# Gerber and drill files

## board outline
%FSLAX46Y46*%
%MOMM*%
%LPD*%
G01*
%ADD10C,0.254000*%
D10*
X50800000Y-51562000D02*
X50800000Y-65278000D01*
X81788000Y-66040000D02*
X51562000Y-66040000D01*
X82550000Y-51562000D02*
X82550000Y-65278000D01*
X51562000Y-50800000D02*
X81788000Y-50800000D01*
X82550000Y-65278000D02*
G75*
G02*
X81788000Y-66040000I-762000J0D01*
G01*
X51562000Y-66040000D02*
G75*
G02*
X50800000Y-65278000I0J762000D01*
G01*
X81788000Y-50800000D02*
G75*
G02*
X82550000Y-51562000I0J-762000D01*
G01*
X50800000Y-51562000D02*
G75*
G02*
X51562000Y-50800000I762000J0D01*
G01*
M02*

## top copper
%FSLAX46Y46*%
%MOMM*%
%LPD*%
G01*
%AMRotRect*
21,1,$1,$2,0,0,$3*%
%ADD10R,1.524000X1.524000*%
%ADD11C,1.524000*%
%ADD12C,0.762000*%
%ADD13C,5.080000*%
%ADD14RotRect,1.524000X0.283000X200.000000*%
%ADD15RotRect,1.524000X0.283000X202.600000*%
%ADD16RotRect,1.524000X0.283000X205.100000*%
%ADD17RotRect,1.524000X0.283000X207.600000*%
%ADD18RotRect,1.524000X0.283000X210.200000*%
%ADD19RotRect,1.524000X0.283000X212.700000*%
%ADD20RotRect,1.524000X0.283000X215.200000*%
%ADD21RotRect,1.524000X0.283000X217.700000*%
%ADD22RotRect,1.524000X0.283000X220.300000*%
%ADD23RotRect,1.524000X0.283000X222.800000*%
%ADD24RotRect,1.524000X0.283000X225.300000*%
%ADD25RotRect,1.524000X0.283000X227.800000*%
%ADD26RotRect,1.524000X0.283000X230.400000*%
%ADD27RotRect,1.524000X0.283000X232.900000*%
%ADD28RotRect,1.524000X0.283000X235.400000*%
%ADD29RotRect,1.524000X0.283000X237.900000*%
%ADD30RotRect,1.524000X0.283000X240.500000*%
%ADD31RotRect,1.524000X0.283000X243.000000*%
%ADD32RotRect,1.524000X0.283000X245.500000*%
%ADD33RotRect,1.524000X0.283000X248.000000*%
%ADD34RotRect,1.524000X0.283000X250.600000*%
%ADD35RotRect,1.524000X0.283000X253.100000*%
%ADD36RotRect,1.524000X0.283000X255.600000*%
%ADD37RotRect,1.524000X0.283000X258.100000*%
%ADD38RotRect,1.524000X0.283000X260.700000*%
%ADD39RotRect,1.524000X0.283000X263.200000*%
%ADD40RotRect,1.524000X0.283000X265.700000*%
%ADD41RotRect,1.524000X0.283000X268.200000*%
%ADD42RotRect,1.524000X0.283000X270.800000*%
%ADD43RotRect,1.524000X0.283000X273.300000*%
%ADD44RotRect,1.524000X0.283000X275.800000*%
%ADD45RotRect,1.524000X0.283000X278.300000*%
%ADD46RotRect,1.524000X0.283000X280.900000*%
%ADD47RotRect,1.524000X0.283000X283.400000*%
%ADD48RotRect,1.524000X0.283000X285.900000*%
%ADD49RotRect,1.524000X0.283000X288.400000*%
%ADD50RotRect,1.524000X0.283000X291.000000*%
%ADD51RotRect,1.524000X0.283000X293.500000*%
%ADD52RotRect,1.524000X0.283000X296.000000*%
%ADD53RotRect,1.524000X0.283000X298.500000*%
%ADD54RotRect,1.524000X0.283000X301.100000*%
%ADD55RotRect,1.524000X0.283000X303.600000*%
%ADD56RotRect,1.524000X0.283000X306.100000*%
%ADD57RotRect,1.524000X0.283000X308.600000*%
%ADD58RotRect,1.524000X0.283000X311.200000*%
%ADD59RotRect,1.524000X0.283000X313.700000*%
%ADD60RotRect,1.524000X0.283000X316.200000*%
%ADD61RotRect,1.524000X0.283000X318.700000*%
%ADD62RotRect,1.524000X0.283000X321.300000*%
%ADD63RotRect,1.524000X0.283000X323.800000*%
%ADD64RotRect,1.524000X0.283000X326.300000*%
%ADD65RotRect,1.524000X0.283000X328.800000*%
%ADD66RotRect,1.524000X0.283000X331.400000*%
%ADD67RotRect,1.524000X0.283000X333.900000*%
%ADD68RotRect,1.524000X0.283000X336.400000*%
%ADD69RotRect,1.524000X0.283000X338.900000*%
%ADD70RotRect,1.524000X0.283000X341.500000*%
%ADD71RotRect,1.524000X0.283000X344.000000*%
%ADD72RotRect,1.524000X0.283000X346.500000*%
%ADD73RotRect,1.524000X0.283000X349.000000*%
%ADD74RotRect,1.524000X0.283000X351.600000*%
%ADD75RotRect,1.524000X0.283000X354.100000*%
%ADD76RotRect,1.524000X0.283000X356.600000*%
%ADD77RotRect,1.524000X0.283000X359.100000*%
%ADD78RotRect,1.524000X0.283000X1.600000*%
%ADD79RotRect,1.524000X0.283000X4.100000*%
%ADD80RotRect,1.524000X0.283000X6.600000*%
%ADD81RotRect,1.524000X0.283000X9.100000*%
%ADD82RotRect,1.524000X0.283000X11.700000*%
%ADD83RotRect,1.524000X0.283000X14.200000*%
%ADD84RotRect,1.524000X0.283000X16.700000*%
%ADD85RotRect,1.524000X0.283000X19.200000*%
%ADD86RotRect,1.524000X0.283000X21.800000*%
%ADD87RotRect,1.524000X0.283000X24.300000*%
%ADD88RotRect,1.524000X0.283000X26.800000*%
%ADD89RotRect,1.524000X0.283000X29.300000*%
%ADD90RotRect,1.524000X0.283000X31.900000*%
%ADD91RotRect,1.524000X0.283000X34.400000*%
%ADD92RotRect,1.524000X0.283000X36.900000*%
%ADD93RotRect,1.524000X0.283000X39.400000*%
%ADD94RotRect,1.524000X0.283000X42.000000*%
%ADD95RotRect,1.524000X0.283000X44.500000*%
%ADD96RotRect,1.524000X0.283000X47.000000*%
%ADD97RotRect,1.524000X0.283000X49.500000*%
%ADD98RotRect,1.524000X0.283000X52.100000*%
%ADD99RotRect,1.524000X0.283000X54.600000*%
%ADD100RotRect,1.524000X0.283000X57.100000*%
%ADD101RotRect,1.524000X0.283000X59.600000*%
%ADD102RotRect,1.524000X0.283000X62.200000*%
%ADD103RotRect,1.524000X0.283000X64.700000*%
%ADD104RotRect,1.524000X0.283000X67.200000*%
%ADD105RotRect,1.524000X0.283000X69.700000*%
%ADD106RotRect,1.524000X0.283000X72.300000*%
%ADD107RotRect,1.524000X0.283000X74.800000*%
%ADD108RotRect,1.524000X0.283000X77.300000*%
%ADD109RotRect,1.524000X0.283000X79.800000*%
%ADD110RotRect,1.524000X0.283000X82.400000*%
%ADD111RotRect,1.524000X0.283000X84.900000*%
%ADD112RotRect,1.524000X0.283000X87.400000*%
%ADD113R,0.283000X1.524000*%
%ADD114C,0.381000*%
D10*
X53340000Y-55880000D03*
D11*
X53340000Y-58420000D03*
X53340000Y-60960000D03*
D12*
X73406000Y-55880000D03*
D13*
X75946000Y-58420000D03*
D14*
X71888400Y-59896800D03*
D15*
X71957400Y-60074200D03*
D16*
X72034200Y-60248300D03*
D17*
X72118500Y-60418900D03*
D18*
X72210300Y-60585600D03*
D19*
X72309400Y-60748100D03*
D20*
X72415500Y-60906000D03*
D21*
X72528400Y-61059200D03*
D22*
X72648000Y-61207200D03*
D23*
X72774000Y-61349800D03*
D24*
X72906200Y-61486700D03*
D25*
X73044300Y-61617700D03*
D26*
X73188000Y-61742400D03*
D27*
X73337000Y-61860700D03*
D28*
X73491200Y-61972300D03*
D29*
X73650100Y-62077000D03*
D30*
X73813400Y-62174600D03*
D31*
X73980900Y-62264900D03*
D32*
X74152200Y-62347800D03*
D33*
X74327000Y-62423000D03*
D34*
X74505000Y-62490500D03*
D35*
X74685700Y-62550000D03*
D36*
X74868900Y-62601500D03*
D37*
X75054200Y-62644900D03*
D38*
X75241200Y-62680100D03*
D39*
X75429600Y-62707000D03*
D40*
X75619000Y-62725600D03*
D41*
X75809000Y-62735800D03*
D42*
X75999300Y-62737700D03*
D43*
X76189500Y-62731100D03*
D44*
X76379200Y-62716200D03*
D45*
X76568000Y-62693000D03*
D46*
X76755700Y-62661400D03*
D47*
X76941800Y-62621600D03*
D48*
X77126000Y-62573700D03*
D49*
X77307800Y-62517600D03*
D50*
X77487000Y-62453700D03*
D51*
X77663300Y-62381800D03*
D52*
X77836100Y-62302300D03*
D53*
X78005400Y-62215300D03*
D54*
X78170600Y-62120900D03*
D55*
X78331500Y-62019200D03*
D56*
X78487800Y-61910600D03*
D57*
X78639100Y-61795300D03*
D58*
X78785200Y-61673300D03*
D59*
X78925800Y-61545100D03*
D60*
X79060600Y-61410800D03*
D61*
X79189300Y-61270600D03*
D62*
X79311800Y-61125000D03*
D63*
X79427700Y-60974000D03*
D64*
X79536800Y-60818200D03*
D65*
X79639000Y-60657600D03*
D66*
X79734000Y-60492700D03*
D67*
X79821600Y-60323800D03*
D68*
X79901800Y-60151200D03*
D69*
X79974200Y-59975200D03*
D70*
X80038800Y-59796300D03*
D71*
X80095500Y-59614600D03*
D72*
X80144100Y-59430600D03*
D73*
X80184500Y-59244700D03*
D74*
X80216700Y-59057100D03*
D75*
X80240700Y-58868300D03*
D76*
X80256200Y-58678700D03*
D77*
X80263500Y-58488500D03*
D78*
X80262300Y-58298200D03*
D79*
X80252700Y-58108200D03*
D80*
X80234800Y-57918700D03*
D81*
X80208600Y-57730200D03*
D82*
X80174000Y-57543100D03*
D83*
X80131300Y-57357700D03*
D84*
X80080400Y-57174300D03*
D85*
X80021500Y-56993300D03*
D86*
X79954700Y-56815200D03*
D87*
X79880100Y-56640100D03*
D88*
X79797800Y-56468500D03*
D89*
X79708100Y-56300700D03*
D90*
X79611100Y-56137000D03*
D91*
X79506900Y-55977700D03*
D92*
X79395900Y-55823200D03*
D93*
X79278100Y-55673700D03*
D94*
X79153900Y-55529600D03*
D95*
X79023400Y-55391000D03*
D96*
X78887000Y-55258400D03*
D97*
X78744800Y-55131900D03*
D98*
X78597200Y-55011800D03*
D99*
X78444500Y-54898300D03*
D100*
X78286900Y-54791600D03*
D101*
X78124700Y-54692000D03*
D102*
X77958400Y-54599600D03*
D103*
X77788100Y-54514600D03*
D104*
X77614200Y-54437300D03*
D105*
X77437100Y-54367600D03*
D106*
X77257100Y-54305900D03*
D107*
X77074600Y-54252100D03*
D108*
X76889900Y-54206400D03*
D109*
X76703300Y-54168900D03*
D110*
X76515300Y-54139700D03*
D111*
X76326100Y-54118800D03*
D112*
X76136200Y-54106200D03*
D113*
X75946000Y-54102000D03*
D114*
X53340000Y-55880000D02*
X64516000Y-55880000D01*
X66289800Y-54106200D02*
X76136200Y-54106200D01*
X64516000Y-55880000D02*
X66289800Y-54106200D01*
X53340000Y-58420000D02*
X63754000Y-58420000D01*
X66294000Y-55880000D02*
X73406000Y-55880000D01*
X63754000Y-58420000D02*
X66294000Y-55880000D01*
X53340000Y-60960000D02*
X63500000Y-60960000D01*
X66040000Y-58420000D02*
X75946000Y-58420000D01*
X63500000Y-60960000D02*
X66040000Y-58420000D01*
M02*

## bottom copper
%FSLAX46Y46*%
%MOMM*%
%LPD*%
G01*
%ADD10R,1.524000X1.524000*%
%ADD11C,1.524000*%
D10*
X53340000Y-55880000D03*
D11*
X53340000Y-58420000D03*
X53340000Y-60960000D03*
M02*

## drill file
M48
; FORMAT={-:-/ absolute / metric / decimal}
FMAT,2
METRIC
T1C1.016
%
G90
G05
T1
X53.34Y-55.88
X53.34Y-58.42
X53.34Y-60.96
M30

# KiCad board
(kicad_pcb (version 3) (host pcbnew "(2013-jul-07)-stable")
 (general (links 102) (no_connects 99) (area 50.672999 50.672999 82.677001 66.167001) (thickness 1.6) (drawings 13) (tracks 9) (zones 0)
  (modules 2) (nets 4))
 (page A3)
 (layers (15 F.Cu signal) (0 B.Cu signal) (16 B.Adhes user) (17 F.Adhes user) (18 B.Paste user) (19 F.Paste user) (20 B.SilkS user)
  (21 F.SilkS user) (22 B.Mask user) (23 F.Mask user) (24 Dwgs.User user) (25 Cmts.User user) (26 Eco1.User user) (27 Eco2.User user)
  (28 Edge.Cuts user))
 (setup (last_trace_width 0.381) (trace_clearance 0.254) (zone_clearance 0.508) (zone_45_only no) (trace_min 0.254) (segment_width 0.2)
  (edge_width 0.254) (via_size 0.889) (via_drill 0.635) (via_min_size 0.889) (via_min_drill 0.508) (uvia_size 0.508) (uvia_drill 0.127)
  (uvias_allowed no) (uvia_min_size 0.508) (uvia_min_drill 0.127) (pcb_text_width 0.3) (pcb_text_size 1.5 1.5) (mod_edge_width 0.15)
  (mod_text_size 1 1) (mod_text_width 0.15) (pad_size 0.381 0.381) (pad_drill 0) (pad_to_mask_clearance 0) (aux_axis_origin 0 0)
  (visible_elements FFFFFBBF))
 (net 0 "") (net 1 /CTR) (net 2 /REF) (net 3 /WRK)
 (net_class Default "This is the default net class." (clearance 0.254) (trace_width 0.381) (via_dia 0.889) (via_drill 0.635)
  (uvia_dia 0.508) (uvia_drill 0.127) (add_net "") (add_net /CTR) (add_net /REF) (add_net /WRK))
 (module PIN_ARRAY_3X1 (layer F.Cu) (at 53.34 58.42 270)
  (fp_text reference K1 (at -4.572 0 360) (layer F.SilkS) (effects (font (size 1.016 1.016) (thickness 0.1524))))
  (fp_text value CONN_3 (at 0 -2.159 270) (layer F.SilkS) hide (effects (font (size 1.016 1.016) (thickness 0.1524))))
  (pad 1 thru_hole rect (at -2.54 0 270) (size 1.524 1.524) (drill 1.016) (layers *.Cu *.Mask F.SilkS) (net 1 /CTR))
  (pad 2 thru_hole circle (at 0 0 270) (size 1.524 1.524) (drill 1.016) (layers *.Cu *.Mask F.SilkS) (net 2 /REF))
  (pad 3 thru_hole circle (at 2.54 0 270) (size 1.524 1.524) (drill 1.016) (layers *.Cu *.Mask F.SilkS) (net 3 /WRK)))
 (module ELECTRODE (layer F.Cu) (at 75.946 58.42)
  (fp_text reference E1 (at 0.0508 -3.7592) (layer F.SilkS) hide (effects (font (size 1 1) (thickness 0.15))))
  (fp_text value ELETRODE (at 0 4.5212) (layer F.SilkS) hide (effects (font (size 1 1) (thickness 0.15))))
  (pad 1 smd circle (at -2.54 -2.54 225) (size 0.762 0.762) (layers F.Cu F.Paste F.Mask) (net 2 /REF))
  (pad 2 smd circle (at 0 0) (size 5.08 5.08) (layers F.Cu F.Paste F.Mask) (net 3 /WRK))
  (pad 3 smd rect (at -4.0576 1.4768 200) (size 1.524 0.283) (layers F.Cu F.Paste F.Mask) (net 1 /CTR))
  (pad 3 smd rect (at -3.9886 1.6542 202.6) (size 1.524 0.283) (layers F.Cu F.Paste F.Mask) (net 1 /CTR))
  (pad 3 smd rect (at -3.9118 1.8283 205.1) (size 1.524 0.283) (layers F.Cu F.Paste F.Mask) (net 1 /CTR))
  (pad 3 smd rect (at -3.8275 1.9989 207.6) (size 1.524 0.283) (layers F.Cu F.Paste F.Mask) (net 1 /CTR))
  (pad 3 smd rect (at -3.7357 2.1656 210.2) (size 1.524 0.283) (layers F.Cu F.Paste F.Mask) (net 1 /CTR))
  (pad 3 smd rect (at -3.6366 2.3281 212.7) (size 1.524 0.283) (layers F.Cu F.Paste F.Mask) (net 1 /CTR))
  (pad 3 smd rect (at -3.5305 2.486 215.2) (size 1.524 0.283) (layers F.Cu F.Paste F.Mask) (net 1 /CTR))
  (pad 3 smd rect (at -3.4176 2.6392 217.7) (size 1.524 0.283) (layers F.Cu F.Paste F.Mask) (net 1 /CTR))
  (pad 3 smd rect (at -3.298 2.7872 220.3) (size 1.524 0.283) (layers F.Cu F.Paste F.Mask) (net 1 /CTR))
  (pad 3 smd rect (at -3.172 2.9298 222.8) (size 1.524 0.283) (layers F.Cu F.Paste F.Mask) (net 1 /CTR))
  (pad 3 smd rect (at -3.0398 3.0667 225.3) (size 1.524 0.283) (layers F.Cu F.Paste F.Mask) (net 1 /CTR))
  (pad 3 smd rect (at -2.9017 3.1977 227.8) (size 1.524 0.283) (layers F.Cu F.Paste F.Mask) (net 1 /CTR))
  (pad 3 smd rect (at -2.758 3.3224 230.4) (size 1.524 0.283) (layers F.Cu F.Paste F.Mask) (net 1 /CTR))
  (pad 3 smd rect (at -2.609 3.4407 232.9) (size 1.524 0.283) (layers F.Cu F.Paste F.Mask) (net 1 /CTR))
  (pad 3 smd rect (at -2.4548 3.5523 235.4) (size 1.524 0.283) (layers F.Cu F.Paste F.Mask) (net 1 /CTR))
  (pad 3 smd rect (at -2.2959 3.657 237.9) (size 1.524 0.283) (layers F.Cu F.Paste F.Mask) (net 1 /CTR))
  (pad 3 smd rect (at -2.1326 3.7546 240.5) (size 1.524 0.283) (layers F.Cu F.Paste F.Mask) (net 1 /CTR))
  (pad 3 smd rect (at -1.9651 3.8449 243) (size 1.524 0.283) (layers F.Cu F.Paste F.Mask) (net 1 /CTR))
  (pad 3 smd rect (at -1.7938 3.9278 245.5) (size 1.524 0.283) (layers F.Cu F.Paste F.Mask) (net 1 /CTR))
  (pad 3 smd rect (at -1.619 4.003 248) (size 1.524 0.283) (layers F.Cu F.Paste F.Mask) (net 1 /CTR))
  (pad 3 smd rect (at -1.441 4.0705 250.6) (size 1.524 0.283) (layers F.Cu F.Paste F.Mask) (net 1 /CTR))
  (pad 3 smd rect (at -1.2603 4.13 253.1) (size 1.524 0.283) (layers F.Cu F.Paste F.Mask) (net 1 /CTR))
  (pad 3 smd rect (at -1.0771 4.1815 255.6) (size 1.524 0.283) (layers F.Cu F.Paste F.Mask) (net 1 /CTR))
  (pad 3 smd rect (at -0.8918 4.2249 258.1) (size 1.524 0.283) (layers F.Cu F.Paste F.Mask) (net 1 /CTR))
  (pad 3 smd rect (at -0.7048 4.2601 260.7) (size 1.524 0.283) (layers F.Cu F.Paste F.Mask) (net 1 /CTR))
  (pad 3 smd rect (at -0.5164 4.287 263.2) (size 1.524 0.283) (layers F.Cu F.Paste F.Mask) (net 1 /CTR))
  (pad 3 smd rect (at -0.327 4.3056 265.7) (size 1.524 0.283) (layers F.Cu F.Paste F.Mask) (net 1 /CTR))
  (pad 3 smd rect (at -0.137 4.3158 268.2) (size 1.524 0.283) (layers F.Cu F.Paste F.Mask) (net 1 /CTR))
  (pad 3 smd rect (at 0.0533 4.3177 270.8) (size 1.524 0.283) (layers F.Cu F.Paste F.Mask) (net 1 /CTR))
  (pad 3 smd rect (at 0.2435 4.3111 273.3) (size 1.524 0.283) (layers F.Cu F.Paste F.Mask) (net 1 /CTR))
  (pad 3 smd rect (at 0.4332 4.2962 275.8) (size 1.524 0.283) (layers F.Cu F.Paste F.Mask) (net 1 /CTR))
  (pad 3 smd rect (at 0.622 4.273 278.3) (size 1.524 0.283) (layers F.Cu F.Paste F.Mask) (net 1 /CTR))
  (pad 3 smd rect (at 0.8097 4.2414 280.9) (size 1.524 0.283) (layers F.Cu F.Paste F.Mask) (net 1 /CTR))
  (pad 3 smd rect (at 0.9958 4.2016 283.4) (size 1.524 0.283) (layers F.Cu F.Paste F.Mask) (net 1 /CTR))
  (pad 3 smd rect (at 1.18 4.1537 285.9) (size 1.524 0.283) (layers F.Cu F.Paste F.Mask) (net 1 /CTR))
  (pad 3 smd rect (at 1.3618 4.0976 288.4) (size 1.524 0.283) (layers F.Cu F.Paste F.Mask) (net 1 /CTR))
  (pad 3 smd rect (at 1.541 4.0337 291) (size 1.524 0.283) (layers F.Cu F.Paste F.Mask) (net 1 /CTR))
  (pad 3 smd rect (at 1.7173 3.9618 293.5) (size 1.524 0.283) (layers F.Cu F.Paste F.Mask) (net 1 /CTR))
  (pad 3 smd rect (at 1.8901 3.8823 296) (size 1.524 0.283) (layers F.Cu F.Paste F.Mask) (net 1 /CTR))
  (pad 3 smd rect (at 2.0594 3.7953 298.5) (size 1.524 0.283) (layers F.Cu F.Paste F.Mask) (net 1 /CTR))
  (pad 3 smd rect (at 2.2246 3.7009 301.1) (size 1.524 0.283) (layers F.Cu F.Paste F.Mask) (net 1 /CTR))
  (pad 3 smd rect (at 2.3855 3.5992 303.6) (size 1.524 0.283) (layers F.Cu F.Paste F.Mask) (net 1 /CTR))
  (pad 3 smd rect (at 2.5418 3.4906 306.1) (size 1.524 0.283) (layers F.Cu F.Paste F.Mask) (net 1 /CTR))
  (pad 3 smd rect (at 2.6931 3.3753 308.6) (size 1.524 0.283) (layers F.Cu F.Paste F.Mask) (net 1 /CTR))
  (pad 3 smd rect (at 2.8392 3.2533 311.2) (size 1.524 0.283) (layers F.Cu F.Paste F.Mask) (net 1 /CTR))
  (pad 3 smd rect (at 2.9798 3.1251 313.7) (size 1.524 0.283) (layers F.Cu F.Paste F.Mask) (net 1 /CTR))
  (pad 3 smd rect (at 3.1146 2.9908 316.2) (size 1.524 0.283) (layers F.Cu F.Paste F.Mask) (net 1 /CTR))
  (pad 3 smd rect (at 3.2433 2.8506 318.7) (size 1.524 0.283) (layers F.Cu F.Paste F.Mask) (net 1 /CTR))
  (pad 3 smd rect (at 3.3658 2.705 321.3) (size 1.524 0.283) (layers F.Cu F.Paste F.Mask) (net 1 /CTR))
  (pad 3 smd rect (at 3.4817 2.554 323.8) (size 1.524 0.283) (layers F.Cu F.Paste F.Mask) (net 1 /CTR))
  (pad 3 smd rect (at 3.5908 2.3982 326.3) (size 1.524 0.283) (layers F.Cu F.Paste F.Mask) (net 1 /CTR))
  (pad 3 smd rect (at 3.693 2.2376 328.8) (size 1.524 0.283) (layers F.Cu F.Paste F.Mask) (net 1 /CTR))
  (pad 3 smd rect (at 3.788 2.0727 331.4) (size 1.524 0.283) (layers F.Cu F.Paste F.Mask) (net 1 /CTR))
  (pad 3 smd rect (at 3.8756 1.9038 333.9) (size 1.524 0.283) (layers F.Cu F.Paste F.Mask) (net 1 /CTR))
  (pad 3 smd rect (at 3.9558 1.7312 336.4) (size 1.524 0.283) (layers F.Cu F.Paste F.Mask) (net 1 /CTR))
  (pad 3 smd rect (at 4.0282 1.5552 338.9) (size 1.524 0.283) (layers F.Cu F.Paste F.Mask) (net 1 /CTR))
  (pad 3 smd rect (at 4.0928 1.3763 341.5) (size 1.524 0.283) (layers F.Cu F.Paste F.Mask) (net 1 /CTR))
  (pad 3 smd rect (at 4.1495 1.1946 344) (size 1.524 0.283) (layers F.Cu F.Paste F.Mask) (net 1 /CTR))
  (pad 3 smd rect (at 4.1981 1.0106 346.5) (size 1.524 0.283) (layers F.Cu F.Paste F.Mask) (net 1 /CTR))
  (pad 3 smd rect (at 4.2385 0.8247 349) (size 1.524 0.283) (layers F.Cu F.Paste F.Mask) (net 1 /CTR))
  (pad 3 smd rect (at 4.2707 0.6371 351.6) (size 1.524 0.283) (layers F.Cu F.Paste F.Mask) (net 1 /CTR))
  (pad 3 smd rect (at 4.2947 0.4483 354.1) (size 1.524 0.283) (layers F.Cu F.Paste F.Mask) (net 1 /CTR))
  (pad 3 smd rect (at 4.3102 0.2587 356.6) (size 1.524 0.283) (layers F.Cu F.Paste F.Mask) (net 1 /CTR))
  (pad 3 smd rect (at 4.3175 0.0685 359.1) (size 1.524 0.283) (layers F.Cu F.Paste F.Mask) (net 1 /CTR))
  (pad 3 smd rect (at 4.3163 -0.1218 1.6) (size 1.524 0.283) (layers F.Cu F.Paste F.Mask) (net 1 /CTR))
  (pad 3 smd rect (at 4.3067 -0.3118 4.1) (size 1.524 0.283) (layers F.Cu F.Paste F.Mask) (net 1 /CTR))
  (pad 3 smd rect (at 4.2888 -0.5013 6.6) (size 1.524 0.283) (layers F.Cu F.Paste F.Mask) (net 1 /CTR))
  (pad 3 smd rect (at 4.2626 -0.6898 9.1) (size 1.524 0.283) (layers F.Cu F.Paste F.Mask) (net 1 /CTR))
  (pad 3 smd rect (at 4.228 -0.8769 11.7) (size 1.524 0.283) (layers F.Cu F.Paste F.Mask) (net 1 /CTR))
  (pad 3 smd rect (at 4.1853 -1.0623 14.2) (size 1.524 0.283) (layers F.Cu F.Paste F.Mask) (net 1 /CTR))
  (pad 3 smd rect (at 4.1344 -1.2457 16.7) (size 1.524 0.283) (layers F.Cu F.Paste F.Mask) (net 1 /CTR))
  (pad 3 smd rect (at 4.0755 -1.4267 19.2) (size 1.524 0.283) (layers F.Cu F.Paste F.Mask) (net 1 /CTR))
  (pad 3 smd rect (at 4.0087 -1.6048 21.8) (size 1.524 0.283) (layers F.Cu F.Paste F.Mask) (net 1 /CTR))
  (pad 3 smd rect (at 3.9341 -1.7799 24.3) (size 1.524 0.283) (layers F.Cu F.Paste F.Mask) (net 1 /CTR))
  (pad 3 smd rect (at 3.8518 -1.9515 26.8) (size 1.524 0.283) (layers F.Cu F.Paste F.Mask) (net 1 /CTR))
  (pad 3 smd rect (at 3.7621 -2.1193 29.3) (size 1.524 0.283) (layers F.Cu F.Paste F.Mask) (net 1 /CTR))
  (pad 3 smd rect (at 3.6651 -2.283 31.9) (size 1.524 0.283) (layers F.Cu F.Paste F.Mask) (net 1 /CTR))
  (pad 3 smd rect (at 3.5609 -2.4423 34.4) (size 1.524 0.283) (layers F.Cu F.Paste F.Mask) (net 1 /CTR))
  (pad 3 smd rect (at 3.4499 -2.5968 36.9) (size 1.524 0.283) (layers F.Cu F.Paste F.Mask) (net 1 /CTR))
  (pad 3 smd rect (at 3.3321 -2.7463 39.4) (size 1.524 0.283) (layers F.Cu F.Paste F.Mask) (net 1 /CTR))
  (pad 3 smd rect (at 3.2079 -2.8904 42) (size 1.524 0.283) (layers F.Cu F.Paste F.Mask) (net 1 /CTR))
  (pad 3 smd rect (at 3.0774 -3.029 44.5) (size 1.524 0.283) (layers F.Cu F.Paste F.Mask) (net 1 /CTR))
  (pad 3 smd rect (at 2.941 -3.1616 47) (size 1.524 0.283) (layers F.Cu F.Paste F.Mask) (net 1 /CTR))
  (pad 3 smd rect (at 2.7988 -3.2881 49.5) (size 1.524 0.283) (layers F.Cu F.Paste F.Mask) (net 1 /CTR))
  (pad 3 smd rect (at 2.6512 -3.4082 52.1) (size 1.524 0.283) (layers F.Cu F.Paste F.Mask) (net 1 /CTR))
  (pad 3 smd rect (at 2.4985 -3.5217 54.6) (size 1.524 0.283) (layers F.Cu F.Paste F.Mask) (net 1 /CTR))
  (pad 3 smd rect (at 2.3409 -3.6284 57.1) (size 1.524 0.283) (layers F.Cu F.Paste F.Mask) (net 1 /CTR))
  (pad 3 smd rect (at 2.1787 -3.728 59.6) (size 1.524 0.283) (layers F.Cu F.Paste F.Mask) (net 1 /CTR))
  (pad 3 smd rect (at 2.0124 -3.8204 62.2) (size 1.524 0.283) (layers F.Cu F.Paste F.Mask) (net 1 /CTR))
  (pad 3 smd rect (at 1.8421 -3.9054 64.7) (size 1.524 0.283) (layers F.Cu F.Paste F.Mask) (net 1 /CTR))
  (pad 3 smd rect (at 1.6682 -3.9827 67.2) (size 1.524 0.283) (layers F.Cu F.Paste F.Mask) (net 1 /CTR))
  (pad 3 smd rect (at 1.4911 -4.0524 69.7) (size 1.524 0.283) (layers F.Cu F.Paste F.Mask) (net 1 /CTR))
  (pad 3 smd rect (at 1.3111 -4.1141 72.3) (size 1.524 0.283) (layers F.Cu F.Paste F.Mask) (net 1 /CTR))
  (pad 3 smd rect (at 1.1286 -4.1679 74.8) (size 1.524 0.283) (layers F.Cu F.Paste F.Mask) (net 1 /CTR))
  (pad 3 smd rect (at 0.9439 -4.2136 77.3) (size 1.524 0.283) (layers F.Cu F.Paste F.Mask) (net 1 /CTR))
  (pad 3 smd rect (at 0.7573 -4.2511 79.8) (size 1.524 0.283) (layers F.Cu F.Paste F.Mask) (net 1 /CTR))
  (pad 3 smd rect (at 0.5693 -4.2803 82.4) (size 1.524 0.283) (layers F.Cu F.Paste F.Mask) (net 1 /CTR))
  (pad 3 smd rect (at 0.3801 -4.3012 84.9) (size 1.524 0.283) (layers F.Cu F.Paste F.Mask) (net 1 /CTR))
  (pad 3 smd rect (at 0.1902 -4.3138 87.4) (size 1.524 0.283) (layers F.Cu F.Paste F.Mask) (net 1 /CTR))
  (pad 3 smd rect (at 0 -4.318 90) (size 1.524 0.283) (layers F.Cu F.Paste F.Mask) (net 1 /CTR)))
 (gr_line (start 50.8 51.562) (end 50.8 65.278) (angle 90) (layer Edge.Cuts) (width 0.254))
 (gr_line (start 81.788 66.04) (end 51.562 66.04) (angle 90) (layer Edge.Cuts) (width 0.254))
 (gr_line (start 82.55 51.562) (end 82.55 65.278) (angle 90) (layer Edge.Cuts) (width 0.254))
 (gr_line (start 51.562 50.8) (end 81.788 50.8) (angle 90) (layer Edge.Cuts) (width 0.254))
 (gr_arc (start 81.788 65.278) (end 82.55 65.278) (angle 90) (layer Edge.Cuts) (width 0.254))
 (gr_arc (start 51.562 65.278) (end 51.562 66.04) (angle 90) (layer Edge.Cuts) (width 0.254))
 (gr_arc (start 81.788 51.562) (end 81.788 50.8) (angle 90) (layer Edge.Cuts) (width 0.254))
 (gr_arc (start 51.562 51.562) (end 50.8 51.562) (angle 90) (layer Edge.Cuts) (width 0.254))
 (segment (start 53.34 55.88) (end 64.516 55.88) (width 0.381) (layer F.Cu) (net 1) (status 400000))
 (segment (start 66.2898 54.1062) (end 76.1362 54.1062) (width 0.381) (layer F.Cu) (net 1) (status 800000))
 (segment (start 64.516 55.88) (end 66.2898 54.1062) (width 0.381) (layer F.Cu) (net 1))
 (segment (start 53.34 58.42) (end 63.754 58.42) (width 0.381) (layer F.Cu) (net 2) (status 400000))
 (segment (start 66.294 55.88) (end 73.406 55.88) (width 0.381) (layer F.Cu) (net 2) (status 800000))
 (segment (start 63.754 58.42) (end 66.294 55.88) (width 0.381) (layer F.Cu) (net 2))
 (segment (start 53.34 60.96) (end 63.5 60.96) (width 0.381) (layer F.Cu) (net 3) (status 400000))
 (segment (start 66.04 58.42) (end 75.946 58.42) (width 0.381) (layer F.Cu) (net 3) (status 800000))
 (segment (start 63.5 60.96) (end 66.04 58.42) (width 0.381) (layer F.Cu) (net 3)))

